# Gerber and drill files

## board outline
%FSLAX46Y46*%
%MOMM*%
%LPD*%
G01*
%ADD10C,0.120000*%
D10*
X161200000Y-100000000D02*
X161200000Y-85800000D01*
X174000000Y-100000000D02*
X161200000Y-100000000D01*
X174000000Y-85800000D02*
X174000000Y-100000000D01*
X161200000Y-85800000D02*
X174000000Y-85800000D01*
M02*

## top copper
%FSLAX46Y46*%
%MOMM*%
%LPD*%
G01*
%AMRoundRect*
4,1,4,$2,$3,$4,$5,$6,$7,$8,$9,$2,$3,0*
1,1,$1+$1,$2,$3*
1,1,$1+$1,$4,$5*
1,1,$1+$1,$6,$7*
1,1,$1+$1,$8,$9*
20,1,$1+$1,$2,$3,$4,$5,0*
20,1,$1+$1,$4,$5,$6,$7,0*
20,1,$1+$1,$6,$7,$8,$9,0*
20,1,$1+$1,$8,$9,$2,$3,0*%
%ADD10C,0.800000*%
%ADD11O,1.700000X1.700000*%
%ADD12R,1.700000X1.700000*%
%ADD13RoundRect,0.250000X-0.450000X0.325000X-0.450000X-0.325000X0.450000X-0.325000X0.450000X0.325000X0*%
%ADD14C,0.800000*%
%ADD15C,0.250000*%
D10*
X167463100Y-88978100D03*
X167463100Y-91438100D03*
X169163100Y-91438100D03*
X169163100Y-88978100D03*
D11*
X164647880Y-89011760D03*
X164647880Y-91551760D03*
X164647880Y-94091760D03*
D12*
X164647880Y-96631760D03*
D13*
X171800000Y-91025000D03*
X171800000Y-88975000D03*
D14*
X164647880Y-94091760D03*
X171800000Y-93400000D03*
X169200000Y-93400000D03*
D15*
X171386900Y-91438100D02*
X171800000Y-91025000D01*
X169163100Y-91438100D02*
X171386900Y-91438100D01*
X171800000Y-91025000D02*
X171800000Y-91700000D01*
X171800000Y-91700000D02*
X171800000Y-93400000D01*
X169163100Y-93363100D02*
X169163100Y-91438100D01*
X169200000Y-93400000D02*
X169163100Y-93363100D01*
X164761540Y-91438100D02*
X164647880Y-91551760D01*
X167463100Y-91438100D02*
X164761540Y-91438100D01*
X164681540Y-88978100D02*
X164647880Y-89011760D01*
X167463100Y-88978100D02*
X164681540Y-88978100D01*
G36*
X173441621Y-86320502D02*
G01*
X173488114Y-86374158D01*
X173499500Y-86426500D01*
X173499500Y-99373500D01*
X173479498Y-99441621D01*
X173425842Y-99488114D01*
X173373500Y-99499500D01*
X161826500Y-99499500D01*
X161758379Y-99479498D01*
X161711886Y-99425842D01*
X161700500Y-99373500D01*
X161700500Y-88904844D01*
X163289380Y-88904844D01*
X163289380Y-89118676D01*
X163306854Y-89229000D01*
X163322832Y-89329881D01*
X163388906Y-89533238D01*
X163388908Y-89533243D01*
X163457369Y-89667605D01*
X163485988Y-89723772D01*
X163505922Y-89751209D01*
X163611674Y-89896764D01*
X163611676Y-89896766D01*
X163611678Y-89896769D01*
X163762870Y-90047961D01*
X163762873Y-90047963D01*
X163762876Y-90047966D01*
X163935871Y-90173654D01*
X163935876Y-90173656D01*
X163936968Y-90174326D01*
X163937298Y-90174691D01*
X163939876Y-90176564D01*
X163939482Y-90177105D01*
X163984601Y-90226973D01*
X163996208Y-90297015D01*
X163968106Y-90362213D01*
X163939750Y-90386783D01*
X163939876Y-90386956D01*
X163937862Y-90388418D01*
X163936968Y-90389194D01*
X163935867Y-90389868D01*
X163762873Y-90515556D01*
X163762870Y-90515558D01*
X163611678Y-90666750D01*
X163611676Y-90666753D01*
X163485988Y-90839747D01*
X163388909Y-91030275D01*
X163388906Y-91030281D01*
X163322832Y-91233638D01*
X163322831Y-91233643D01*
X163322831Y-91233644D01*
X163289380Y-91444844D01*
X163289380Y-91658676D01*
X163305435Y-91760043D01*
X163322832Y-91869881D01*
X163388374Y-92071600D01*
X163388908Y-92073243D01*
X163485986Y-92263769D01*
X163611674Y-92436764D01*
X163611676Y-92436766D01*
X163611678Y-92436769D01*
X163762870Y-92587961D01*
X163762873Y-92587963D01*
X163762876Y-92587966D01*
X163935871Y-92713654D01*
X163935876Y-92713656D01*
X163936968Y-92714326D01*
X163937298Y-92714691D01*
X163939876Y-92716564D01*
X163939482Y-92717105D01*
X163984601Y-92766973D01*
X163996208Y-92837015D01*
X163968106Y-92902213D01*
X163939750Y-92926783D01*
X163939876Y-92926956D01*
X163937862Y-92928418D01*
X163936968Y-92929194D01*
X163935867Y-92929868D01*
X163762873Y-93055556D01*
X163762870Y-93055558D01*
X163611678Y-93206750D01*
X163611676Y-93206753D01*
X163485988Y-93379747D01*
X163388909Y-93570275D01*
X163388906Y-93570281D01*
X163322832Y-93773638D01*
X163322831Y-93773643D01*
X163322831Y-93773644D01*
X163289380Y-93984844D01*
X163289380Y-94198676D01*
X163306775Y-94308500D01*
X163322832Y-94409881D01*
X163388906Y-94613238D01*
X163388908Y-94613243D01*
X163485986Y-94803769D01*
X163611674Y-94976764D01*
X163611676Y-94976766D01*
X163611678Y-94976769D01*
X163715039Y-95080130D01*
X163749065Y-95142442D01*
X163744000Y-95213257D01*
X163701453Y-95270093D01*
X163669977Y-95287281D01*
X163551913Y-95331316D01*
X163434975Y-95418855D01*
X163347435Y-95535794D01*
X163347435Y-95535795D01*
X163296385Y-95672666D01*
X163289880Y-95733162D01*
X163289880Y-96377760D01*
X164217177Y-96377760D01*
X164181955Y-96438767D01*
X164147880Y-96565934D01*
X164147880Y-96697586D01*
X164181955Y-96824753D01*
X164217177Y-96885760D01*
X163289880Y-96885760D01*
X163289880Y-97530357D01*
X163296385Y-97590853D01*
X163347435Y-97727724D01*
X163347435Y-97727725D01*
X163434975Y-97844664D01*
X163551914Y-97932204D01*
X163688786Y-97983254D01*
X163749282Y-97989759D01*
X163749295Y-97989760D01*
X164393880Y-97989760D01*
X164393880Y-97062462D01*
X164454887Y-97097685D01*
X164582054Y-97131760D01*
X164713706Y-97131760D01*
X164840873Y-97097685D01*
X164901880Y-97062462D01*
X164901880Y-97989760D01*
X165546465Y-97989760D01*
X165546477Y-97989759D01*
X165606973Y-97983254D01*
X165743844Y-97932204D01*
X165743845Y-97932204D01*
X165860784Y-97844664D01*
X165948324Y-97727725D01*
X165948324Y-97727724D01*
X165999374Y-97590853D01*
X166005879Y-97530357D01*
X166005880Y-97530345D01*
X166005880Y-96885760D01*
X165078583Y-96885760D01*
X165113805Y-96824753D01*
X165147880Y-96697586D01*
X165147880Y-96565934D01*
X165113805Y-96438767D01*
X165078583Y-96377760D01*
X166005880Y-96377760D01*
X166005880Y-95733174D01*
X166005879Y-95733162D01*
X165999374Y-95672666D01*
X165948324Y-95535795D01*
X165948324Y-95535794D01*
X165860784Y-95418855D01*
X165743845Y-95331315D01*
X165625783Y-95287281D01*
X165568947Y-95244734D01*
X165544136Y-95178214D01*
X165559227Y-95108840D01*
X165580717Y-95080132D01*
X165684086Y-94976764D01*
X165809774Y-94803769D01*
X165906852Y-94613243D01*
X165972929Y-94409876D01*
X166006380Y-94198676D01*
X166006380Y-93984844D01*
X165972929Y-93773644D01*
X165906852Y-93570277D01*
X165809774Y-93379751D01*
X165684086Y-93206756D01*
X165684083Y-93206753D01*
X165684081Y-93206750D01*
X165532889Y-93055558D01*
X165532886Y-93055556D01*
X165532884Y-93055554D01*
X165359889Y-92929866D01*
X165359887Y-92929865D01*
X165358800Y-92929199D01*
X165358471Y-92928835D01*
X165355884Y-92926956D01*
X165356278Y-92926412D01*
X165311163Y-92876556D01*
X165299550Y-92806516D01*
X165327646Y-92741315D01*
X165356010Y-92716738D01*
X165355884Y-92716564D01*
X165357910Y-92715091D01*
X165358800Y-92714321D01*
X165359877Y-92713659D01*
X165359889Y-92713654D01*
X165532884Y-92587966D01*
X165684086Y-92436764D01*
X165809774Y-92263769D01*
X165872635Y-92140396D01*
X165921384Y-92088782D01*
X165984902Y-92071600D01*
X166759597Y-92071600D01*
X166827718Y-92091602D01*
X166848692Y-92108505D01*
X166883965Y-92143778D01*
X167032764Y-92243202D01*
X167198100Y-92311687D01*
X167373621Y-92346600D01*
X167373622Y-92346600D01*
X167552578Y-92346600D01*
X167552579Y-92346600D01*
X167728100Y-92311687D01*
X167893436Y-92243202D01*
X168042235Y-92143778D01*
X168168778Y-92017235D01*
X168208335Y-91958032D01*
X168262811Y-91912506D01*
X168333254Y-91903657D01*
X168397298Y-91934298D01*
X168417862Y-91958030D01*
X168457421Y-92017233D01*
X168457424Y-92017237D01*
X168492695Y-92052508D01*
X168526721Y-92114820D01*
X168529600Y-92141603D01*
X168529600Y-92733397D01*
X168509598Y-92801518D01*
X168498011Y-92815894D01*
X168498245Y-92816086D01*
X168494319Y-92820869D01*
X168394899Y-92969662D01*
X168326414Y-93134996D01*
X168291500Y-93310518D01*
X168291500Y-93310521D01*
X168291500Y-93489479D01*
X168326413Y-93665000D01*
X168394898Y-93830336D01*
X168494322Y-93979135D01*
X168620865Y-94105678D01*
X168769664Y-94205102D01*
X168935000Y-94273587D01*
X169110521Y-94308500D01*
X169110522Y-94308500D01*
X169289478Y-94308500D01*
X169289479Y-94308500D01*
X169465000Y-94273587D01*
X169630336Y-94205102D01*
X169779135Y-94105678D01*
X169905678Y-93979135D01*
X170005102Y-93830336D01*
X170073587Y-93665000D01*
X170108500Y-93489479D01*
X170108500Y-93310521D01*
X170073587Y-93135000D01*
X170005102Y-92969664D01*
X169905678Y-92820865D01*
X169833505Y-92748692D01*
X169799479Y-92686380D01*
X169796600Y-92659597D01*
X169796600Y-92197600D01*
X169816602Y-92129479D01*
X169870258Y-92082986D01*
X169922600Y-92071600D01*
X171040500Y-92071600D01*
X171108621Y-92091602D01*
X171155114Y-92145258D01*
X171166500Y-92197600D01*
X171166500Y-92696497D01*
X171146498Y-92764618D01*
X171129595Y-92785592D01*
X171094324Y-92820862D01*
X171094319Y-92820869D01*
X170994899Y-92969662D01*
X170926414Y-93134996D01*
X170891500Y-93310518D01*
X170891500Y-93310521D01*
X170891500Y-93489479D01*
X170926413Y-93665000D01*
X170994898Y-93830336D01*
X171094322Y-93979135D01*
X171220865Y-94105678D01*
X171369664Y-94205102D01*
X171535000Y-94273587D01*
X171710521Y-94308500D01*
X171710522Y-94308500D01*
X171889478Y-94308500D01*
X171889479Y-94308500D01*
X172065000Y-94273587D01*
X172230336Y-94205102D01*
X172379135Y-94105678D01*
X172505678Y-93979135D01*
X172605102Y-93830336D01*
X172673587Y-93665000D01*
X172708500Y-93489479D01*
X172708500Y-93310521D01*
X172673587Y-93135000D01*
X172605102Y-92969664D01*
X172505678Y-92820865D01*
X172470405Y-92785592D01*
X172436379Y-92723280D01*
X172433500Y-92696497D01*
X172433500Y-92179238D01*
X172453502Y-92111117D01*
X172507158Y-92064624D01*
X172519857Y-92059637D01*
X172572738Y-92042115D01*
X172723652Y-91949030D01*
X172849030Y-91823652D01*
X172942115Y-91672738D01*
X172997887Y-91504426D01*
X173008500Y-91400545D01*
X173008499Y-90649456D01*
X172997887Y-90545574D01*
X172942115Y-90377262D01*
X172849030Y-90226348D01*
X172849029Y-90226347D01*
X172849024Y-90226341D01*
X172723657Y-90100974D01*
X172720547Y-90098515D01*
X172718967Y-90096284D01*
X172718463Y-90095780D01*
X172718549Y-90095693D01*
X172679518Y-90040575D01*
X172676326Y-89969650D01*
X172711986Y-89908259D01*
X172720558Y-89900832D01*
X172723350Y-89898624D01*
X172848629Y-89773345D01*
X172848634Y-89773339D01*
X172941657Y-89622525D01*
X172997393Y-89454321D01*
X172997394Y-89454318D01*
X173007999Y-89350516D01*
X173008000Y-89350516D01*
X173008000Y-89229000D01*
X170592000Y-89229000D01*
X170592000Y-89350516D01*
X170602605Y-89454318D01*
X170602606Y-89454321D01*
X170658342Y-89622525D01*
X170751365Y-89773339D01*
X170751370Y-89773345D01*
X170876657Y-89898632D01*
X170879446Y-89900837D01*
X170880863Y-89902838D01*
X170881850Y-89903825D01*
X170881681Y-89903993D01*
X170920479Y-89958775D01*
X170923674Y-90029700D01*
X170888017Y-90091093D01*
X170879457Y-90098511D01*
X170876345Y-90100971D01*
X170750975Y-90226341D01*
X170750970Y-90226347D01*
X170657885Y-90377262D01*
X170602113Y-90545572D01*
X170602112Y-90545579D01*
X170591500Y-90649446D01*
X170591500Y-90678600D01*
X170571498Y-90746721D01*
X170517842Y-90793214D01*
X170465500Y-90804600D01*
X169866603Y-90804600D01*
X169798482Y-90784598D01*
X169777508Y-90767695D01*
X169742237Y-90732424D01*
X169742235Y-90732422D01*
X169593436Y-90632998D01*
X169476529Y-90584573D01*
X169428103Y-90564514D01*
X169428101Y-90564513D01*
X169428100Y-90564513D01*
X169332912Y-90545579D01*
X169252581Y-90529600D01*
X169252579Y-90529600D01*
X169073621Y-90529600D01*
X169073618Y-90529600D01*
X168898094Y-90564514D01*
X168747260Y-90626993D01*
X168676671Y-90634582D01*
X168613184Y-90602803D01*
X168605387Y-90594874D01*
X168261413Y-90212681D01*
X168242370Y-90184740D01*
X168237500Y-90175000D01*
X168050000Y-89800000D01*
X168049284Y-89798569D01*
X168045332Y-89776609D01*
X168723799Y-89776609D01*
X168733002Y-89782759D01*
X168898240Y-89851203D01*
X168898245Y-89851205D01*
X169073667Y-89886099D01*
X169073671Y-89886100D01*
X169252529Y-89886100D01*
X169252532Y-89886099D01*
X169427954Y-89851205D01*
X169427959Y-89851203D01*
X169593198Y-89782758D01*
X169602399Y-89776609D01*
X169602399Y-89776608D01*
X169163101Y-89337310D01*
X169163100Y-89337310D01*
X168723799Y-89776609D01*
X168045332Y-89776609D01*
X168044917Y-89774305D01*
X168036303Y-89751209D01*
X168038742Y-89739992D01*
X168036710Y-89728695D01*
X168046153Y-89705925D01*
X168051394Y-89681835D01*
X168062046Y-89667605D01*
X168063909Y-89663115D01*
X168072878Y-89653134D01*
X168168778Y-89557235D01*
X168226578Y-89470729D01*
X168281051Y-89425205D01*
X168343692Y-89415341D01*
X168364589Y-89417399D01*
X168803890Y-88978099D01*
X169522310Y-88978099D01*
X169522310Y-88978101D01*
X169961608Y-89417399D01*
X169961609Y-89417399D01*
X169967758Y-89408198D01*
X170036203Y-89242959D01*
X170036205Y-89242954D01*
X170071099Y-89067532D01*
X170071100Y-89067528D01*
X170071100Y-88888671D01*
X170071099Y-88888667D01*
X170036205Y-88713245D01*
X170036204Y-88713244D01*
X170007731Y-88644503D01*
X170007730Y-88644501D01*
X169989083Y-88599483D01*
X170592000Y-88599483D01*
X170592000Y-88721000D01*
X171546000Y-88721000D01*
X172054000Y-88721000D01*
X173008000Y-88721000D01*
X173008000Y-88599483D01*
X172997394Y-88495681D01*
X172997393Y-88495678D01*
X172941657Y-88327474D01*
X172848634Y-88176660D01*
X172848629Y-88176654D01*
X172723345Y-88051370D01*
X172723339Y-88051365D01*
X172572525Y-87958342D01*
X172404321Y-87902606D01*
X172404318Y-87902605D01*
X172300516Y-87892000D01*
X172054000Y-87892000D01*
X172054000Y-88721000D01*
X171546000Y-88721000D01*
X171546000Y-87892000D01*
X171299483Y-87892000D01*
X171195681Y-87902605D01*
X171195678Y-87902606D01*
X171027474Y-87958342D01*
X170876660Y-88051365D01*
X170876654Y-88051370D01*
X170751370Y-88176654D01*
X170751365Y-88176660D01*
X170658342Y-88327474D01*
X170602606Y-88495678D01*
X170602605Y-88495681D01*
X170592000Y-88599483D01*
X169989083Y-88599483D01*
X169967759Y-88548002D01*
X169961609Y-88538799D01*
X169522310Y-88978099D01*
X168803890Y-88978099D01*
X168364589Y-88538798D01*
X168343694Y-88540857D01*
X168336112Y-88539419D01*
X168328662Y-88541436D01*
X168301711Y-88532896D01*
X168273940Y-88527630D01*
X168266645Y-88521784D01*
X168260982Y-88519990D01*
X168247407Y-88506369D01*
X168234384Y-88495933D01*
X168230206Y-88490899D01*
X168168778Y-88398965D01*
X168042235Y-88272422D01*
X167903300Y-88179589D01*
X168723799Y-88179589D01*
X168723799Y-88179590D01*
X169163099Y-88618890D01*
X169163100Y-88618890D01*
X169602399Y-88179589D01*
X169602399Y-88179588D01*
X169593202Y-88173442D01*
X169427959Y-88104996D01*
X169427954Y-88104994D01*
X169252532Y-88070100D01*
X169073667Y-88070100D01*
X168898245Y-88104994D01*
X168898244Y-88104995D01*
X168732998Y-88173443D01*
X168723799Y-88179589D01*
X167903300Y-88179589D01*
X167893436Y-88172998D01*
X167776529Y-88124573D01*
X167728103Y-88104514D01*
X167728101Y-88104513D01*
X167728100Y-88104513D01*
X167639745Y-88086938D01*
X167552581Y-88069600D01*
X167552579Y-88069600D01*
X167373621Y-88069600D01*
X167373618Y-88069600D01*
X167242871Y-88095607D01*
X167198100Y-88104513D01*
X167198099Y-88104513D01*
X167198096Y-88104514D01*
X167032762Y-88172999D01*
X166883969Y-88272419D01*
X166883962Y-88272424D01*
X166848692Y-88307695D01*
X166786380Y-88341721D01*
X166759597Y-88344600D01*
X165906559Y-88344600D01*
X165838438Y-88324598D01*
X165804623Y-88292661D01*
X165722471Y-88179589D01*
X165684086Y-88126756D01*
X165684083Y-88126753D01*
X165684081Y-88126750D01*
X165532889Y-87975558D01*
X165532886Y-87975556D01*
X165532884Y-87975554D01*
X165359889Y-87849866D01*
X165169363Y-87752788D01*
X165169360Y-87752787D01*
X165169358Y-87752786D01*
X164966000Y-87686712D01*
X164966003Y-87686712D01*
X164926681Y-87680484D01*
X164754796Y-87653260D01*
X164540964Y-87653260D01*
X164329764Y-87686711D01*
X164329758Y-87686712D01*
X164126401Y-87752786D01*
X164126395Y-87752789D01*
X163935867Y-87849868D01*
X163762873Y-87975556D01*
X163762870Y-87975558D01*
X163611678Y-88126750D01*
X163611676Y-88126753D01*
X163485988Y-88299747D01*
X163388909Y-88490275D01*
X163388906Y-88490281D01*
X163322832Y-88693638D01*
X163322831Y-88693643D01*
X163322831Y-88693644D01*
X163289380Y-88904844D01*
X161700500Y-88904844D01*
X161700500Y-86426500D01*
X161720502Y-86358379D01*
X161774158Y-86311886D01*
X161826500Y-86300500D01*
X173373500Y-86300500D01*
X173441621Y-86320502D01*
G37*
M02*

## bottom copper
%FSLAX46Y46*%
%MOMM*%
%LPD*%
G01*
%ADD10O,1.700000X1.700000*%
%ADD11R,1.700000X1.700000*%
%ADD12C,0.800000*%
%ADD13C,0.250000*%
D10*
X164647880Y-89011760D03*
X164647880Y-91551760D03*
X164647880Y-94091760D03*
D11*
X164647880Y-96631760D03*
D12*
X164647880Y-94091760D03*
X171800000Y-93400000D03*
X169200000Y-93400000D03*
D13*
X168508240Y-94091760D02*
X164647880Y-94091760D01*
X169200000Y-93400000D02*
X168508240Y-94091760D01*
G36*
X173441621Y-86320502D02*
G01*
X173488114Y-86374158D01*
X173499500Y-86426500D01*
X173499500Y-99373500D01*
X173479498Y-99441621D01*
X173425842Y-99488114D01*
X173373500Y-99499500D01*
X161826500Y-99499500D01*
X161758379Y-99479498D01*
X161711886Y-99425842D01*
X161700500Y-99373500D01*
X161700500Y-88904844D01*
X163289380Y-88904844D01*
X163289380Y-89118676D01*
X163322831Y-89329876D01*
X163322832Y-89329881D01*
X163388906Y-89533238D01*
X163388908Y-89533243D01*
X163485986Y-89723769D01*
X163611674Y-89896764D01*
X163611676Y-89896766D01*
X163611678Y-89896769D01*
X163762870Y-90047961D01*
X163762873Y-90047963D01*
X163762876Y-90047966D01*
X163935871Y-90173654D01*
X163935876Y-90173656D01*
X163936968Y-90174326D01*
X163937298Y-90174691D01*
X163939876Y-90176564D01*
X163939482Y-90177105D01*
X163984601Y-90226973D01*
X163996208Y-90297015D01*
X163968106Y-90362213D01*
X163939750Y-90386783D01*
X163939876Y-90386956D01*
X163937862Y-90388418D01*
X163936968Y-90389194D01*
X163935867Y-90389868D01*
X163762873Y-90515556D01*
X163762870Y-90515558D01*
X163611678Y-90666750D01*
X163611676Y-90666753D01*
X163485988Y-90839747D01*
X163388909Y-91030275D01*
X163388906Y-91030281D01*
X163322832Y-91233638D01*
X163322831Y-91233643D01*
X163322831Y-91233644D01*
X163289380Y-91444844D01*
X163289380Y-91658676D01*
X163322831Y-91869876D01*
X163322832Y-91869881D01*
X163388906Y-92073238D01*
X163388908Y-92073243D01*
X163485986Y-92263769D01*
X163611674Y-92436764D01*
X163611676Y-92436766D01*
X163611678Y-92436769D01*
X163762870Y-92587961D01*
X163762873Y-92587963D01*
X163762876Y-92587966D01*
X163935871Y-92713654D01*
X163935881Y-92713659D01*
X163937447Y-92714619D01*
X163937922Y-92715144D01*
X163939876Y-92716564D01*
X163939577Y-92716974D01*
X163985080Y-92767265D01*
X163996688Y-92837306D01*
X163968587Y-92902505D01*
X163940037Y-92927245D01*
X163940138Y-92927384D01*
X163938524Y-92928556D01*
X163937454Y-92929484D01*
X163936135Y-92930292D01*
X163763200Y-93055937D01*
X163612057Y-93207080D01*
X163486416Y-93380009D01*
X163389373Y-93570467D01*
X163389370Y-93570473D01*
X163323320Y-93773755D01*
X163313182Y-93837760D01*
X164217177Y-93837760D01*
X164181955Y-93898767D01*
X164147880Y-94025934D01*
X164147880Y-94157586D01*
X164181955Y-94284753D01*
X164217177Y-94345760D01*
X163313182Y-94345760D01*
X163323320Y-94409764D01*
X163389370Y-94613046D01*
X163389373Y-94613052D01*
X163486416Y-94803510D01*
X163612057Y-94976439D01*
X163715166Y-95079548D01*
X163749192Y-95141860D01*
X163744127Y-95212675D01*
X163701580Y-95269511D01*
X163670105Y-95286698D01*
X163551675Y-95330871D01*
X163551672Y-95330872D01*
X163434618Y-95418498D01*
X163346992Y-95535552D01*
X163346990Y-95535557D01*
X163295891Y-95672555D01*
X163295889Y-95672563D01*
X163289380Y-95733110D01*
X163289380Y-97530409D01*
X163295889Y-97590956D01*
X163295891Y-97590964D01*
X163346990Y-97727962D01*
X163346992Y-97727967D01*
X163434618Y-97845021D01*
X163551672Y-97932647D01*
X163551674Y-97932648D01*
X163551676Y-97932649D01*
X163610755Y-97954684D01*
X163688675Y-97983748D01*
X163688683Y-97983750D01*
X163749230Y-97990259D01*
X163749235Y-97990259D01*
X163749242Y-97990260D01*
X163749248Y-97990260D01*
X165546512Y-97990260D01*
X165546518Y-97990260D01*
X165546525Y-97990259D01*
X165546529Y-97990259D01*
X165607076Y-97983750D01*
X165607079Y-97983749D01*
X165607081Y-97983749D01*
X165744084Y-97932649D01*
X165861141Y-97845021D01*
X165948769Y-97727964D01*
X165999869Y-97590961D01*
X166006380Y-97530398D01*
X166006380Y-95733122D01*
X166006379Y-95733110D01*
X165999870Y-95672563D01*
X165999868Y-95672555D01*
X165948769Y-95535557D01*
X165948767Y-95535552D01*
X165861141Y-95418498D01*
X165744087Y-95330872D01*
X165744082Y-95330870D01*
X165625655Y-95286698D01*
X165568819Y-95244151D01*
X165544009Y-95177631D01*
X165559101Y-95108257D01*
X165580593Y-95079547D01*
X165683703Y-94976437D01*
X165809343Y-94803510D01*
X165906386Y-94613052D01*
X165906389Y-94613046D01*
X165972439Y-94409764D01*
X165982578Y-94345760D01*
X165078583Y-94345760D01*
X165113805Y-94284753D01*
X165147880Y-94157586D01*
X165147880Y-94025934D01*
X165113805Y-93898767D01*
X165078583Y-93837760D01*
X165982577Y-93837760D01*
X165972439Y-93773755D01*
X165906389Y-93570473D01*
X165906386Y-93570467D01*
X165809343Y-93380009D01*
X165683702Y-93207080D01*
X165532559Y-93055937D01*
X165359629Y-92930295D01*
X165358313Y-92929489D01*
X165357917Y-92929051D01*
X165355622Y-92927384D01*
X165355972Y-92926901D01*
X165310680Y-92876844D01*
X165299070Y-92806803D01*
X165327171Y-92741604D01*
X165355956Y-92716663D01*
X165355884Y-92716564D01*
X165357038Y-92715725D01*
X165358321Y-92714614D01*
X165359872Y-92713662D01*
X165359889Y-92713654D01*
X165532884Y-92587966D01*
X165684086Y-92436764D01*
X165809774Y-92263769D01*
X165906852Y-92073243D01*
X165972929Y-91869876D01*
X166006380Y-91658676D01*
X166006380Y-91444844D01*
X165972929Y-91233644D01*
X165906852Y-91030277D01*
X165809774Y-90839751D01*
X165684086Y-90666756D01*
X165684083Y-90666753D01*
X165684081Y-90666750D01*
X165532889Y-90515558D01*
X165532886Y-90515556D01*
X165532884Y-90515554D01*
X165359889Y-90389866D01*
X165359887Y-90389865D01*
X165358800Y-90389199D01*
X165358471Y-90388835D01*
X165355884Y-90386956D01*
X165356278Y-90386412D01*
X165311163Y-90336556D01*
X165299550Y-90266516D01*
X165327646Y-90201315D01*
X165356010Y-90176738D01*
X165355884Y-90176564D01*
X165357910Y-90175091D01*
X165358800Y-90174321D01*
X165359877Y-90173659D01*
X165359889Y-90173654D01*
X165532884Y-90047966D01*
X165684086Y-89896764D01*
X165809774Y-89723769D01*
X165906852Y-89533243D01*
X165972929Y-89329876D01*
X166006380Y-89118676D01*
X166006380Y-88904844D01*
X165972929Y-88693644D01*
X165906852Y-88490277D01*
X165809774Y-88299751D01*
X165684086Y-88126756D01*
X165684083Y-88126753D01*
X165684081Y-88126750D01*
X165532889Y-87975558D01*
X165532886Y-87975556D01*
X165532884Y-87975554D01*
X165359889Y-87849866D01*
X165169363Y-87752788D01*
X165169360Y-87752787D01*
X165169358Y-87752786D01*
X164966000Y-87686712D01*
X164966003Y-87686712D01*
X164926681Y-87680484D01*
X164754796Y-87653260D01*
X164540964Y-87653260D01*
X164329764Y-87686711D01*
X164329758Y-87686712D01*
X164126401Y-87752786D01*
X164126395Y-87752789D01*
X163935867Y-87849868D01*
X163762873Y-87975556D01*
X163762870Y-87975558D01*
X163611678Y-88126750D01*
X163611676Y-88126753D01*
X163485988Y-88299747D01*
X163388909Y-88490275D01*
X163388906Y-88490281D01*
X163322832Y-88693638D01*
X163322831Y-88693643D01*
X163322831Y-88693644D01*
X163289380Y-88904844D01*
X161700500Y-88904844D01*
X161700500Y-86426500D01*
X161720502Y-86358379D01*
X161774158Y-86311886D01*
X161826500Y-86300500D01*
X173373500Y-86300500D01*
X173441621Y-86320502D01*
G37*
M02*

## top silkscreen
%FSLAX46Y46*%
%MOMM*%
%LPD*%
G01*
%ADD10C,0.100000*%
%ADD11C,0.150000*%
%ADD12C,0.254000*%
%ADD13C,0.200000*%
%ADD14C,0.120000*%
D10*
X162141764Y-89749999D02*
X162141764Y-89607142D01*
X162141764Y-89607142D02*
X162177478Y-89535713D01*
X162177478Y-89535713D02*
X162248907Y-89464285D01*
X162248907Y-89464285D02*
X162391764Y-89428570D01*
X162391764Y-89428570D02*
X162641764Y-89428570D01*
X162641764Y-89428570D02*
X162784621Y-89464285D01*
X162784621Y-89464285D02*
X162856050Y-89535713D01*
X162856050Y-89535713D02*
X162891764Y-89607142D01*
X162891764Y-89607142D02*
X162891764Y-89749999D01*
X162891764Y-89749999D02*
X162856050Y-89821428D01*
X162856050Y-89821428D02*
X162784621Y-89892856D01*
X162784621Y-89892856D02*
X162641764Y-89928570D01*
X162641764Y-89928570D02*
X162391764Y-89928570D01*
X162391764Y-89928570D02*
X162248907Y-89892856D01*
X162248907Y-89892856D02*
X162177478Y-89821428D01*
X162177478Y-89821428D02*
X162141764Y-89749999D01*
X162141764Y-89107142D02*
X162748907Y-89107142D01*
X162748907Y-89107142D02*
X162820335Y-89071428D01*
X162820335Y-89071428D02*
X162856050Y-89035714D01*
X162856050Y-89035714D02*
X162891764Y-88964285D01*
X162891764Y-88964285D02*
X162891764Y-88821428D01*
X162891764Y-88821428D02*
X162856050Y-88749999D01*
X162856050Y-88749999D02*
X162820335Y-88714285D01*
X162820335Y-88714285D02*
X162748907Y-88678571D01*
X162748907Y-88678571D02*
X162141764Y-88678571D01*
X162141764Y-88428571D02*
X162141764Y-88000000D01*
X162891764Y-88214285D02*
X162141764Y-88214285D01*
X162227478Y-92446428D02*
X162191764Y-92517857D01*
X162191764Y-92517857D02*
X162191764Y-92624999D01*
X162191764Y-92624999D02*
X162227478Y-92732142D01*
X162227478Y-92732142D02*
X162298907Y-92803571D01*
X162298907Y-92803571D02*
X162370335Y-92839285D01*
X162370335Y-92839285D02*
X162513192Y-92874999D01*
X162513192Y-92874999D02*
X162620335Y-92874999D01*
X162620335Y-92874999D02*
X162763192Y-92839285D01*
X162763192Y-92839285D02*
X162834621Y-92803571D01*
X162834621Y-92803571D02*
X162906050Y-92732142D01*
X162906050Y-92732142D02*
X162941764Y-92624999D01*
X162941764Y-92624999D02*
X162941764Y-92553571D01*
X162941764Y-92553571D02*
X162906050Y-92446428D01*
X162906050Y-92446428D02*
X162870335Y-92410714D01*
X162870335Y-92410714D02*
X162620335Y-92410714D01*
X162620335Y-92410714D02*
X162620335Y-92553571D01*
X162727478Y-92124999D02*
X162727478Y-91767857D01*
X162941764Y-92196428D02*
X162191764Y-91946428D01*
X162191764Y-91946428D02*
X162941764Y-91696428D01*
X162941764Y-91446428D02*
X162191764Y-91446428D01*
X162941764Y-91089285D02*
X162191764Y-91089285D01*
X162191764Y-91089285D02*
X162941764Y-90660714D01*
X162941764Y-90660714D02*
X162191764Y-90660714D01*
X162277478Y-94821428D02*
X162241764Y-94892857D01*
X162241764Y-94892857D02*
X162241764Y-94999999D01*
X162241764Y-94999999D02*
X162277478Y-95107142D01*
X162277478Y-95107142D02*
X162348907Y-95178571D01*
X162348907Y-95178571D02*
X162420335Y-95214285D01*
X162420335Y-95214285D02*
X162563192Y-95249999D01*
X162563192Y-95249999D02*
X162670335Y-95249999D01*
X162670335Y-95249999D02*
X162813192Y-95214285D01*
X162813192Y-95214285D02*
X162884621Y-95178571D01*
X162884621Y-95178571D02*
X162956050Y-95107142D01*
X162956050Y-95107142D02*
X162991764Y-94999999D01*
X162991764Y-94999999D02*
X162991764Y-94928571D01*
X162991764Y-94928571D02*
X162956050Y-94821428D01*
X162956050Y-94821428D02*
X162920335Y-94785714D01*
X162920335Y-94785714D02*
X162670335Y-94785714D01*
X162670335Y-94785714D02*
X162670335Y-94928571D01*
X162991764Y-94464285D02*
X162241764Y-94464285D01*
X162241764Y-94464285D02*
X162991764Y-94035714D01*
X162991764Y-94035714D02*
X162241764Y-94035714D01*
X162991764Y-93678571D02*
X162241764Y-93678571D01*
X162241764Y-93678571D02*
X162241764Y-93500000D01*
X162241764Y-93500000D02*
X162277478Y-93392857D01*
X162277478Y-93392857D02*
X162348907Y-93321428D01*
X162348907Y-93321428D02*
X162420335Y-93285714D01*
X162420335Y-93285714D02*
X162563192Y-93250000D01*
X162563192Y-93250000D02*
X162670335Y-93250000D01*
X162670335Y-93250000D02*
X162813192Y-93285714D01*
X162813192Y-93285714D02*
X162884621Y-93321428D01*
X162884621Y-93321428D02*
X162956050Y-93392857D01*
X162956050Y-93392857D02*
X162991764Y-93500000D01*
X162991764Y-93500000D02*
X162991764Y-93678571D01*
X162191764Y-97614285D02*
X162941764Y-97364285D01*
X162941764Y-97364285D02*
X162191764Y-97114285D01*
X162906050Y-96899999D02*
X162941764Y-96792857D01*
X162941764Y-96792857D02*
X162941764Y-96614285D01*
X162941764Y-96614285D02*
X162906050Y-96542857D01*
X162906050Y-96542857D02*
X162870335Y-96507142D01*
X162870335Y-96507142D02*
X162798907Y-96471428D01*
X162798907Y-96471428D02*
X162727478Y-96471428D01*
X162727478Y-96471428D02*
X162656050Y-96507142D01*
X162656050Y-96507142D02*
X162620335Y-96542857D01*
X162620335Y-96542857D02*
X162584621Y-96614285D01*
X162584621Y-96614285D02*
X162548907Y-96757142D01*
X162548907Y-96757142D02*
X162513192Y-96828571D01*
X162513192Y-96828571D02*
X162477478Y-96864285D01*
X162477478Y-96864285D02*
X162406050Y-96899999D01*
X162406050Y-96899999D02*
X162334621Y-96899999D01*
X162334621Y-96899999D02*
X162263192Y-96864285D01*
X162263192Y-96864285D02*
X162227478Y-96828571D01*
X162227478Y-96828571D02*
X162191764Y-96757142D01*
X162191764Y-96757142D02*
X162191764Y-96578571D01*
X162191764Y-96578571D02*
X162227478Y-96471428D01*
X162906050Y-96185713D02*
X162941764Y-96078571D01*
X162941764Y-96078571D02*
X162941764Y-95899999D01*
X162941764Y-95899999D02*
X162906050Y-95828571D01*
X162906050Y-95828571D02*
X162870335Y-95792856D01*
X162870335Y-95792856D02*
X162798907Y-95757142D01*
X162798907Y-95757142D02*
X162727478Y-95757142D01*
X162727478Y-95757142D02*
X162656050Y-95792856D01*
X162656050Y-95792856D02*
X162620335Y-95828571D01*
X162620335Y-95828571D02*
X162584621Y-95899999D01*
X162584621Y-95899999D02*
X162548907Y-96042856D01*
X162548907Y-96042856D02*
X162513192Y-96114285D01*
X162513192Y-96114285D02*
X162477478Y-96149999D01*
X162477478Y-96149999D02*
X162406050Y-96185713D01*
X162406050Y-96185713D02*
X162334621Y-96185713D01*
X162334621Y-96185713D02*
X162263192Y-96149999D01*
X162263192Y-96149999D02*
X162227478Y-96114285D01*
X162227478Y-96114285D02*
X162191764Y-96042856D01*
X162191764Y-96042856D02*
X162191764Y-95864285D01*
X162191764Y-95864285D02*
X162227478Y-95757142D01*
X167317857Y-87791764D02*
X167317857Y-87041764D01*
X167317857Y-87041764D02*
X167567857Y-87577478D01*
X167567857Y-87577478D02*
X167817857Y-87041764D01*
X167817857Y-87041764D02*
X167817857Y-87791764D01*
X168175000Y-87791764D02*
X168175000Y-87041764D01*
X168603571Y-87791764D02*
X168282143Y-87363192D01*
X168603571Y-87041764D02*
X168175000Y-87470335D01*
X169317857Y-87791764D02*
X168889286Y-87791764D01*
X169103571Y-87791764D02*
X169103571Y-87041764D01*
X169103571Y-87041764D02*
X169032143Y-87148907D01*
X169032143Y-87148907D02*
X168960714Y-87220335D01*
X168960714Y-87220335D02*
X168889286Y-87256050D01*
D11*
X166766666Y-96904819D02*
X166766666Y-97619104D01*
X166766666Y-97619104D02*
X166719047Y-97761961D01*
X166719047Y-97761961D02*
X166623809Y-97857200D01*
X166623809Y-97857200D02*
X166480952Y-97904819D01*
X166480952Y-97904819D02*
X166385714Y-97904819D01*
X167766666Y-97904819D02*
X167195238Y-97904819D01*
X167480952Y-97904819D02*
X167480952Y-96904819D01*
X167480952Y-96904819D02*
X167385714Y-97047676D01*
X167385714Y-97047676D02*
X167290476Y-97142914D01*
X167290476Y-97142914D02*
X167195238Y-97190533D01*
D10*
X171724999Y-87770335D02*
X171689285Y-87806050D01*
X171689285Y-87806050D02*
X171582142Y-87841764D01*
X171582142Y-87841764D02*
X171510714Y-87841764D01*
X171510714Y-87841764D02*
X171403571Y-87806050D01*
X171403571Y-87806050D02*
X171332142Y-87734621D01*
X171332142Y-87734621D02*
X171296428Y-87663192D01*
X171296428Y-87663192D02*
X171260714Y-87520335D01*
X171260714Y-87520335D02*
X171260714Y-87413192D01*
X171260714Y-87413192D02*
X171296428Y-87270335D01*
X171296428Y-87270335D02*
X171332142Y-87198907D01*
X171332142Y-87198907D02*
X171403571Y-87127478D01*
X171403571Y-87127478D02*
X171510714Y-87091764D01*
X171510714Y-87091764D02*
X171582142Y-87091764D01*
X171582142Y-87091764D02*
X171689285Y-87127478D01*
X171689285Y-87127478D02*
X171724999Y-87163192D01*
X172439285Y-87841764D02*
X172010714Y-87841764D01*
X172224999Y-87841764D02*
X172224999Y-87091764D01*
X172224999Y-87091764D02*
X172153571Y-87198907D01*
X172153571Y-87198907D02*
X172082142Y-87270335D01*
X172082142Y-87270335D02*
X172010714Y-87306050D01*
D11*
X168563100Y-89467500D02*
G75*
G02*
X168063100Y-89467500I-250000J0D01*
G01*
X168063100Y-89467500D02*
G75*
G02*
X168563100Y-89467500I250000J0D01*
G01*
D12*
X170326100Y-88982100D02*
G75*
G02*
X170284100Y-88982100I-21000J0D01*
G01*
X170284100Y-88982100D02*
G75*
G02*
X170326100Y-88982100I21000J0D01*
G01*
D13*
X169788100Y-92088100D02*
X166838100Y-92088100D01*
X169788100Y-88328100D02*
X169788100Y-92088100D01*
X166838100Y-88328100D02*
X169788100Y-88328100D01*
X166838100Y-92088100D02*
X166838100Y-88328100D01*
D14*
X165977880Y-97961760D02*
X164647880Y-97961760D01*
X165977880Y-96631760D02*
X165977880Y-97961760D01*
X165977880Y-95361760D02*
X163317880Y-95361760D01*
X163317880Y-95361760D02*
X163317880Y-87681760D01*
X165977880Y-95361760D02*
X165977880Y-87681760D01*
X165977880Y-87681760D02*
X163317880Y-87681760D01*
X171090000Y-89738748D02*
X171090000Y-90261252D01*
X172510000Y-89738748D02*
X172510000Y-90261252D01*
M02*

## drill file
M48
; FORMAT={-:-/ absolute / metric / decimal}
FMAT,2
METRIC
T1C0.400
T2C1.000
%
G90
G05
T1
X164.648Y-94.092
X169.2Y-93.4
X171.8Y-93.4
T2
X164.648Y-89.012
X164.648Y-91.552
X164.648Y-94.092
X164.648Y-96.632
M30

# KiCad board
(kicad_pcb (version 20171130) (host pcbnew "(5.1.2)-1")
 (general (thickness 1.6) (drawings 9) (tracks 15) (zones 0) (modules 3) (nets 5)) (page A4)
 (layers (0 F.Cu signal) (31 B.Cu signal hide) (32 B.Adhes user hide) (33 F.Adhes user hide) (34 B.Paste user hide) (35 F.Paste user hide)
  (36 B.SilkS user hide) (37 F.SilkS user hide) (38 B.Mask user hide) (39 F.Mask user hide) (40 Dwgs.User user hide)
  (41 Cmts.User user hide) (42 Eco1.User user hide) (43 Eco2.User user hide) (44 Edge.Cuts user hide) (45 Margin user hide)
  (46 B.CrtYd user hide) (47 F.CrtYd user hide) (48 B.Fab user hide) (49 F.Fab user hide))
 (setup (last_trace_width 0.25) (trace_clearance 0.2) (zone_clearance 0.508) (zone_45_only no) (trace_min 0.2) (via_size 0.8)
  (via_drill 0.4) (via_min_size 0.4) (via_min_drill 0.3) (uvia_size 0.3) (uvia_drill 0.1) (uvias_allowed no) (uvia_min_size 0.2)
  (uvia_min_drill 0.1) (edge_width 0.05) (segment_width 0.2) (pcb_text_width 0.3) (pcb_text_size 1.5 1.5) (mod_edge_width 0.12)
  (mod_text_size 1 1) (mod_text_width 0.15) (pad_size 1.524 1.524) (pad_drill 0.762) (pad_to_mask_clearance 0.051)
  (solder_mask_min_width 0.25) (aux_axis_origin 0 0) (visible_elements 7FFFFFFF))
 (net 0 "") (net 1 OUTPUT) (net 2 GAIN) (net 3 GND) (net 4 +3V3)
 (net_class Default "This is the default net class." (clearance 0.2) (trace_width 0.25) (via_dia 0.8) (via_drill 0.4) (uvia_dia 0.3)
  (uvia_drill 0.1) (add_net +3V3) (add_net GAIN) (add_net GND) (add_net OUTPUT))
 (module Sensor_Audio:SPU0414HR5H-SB (layer F.Cu) (at 168.3131 90.2081)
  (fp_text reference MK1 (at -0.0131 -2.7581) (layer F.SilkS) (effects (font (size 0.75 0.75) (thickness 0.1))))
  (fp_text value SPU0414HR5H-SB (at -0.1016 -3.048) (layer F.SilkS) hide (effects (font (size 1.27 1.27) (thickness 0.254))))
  (fp_circle (center 0 -0.7406) (end 0.25 -0.7406) (layer F.SilkS) (width 0.15))
  (fp_circle (center 1.992 -1.226) (end 1.971 -1.226) (layer F.SilkS) (width 0.254))
  (fp_line (start 1.475 1.88) (end -1.475 1.88) (layer F.SilkS) (width 0.2))
  (fp_line (start 1.475 -1.88) (end 1.475 1.88) (layer F.SilkS) (width 0.2))
  (fp_line (start -1.475 -1.88) (end 1.475 -1.88) (layer F.SilkS) (width 0.2))
  (fp_line (start -1.475 1.88) (end -1.475 -1.88) (layer F.SilkS) (width 0.2))
  (pad 4 smd circle (at -0.85 -1.23 90) (size 0.8 0.8) (layers F.Cu F.Paste F.Mask) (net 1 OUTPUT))
  (pad 3 smd circle (at -0.85 1.23 90) (size 0.8 0.8) (layers F.Cu F.Paste F.Mask) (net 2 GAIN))
  (pad 2 smd circle (at 0.85 1.23 90) (size 0.8 0.8) (layers F.Cu F.Paste F.Mask) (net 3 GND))
  (pad 1 smd circle (at 0.85 -1.23 90) (size 0.8 0.8) (layers F.Cu F.Paste F.Mask) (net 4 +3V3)))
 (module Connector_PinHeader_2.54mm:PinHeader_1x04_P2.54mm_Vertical (layer F.Cu) (at 164.64788 96.63176 180)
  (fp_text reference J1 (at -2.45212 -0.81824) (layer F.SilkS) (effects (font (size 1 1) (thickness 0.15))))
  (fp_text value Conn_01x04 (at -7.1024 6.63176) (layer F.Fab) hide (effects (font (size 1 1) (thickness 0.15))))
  (fp_line (start -1.33 -1.33) (end 0 -1.33) (layer F.SilkS) (width 0.12))
  (fp_line (start -1.33 0) (end -1.33 -1.33) (layer F.SilkS) (width 0.12))
  (fp_line (start -1.33 1.27) (end 1.33 1.27) (layer F.SilkS) (width 0.12))
  (fp_line (start 1.33 1.27) (end 1.33 8.95) (layer F.SilkS) (width 0.12))
  (fp_line (start -1.33 1.27) (end -1.33 8.95) (layer F.SilkS) (width 0.12))
  (fp_line (start -1.33 8.95) (end 1.33 8.95) (layer F.SilkS) (width 0.12))
  (pad 4 thru_hole oval (at 0 7.62 180) (size 1.7 1.7) (drill 1) (layers *.Cu *.Mask) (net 1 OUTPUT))
  (pad 3 thru_hole oval (at 0 5.08 180) (size 1.7 1.7) (drill 1) (layers *.Cu *.Mask) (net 2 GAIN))
  (pad 2 thru_hole oval (at 0 2.54 180) (size 1.7 1.7) (drill 1) (layers *.Cu *.Mask) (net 3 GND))
  (pad 1 thru_hole rect (at 0 0 180) (size 1.7 1.7) (drill 1) (layers *.Cu *.Mask) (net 4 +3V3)))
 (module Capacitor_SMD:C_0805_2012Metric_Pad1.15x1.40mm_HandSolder (layer F.Cu) (at 171.8 90 270)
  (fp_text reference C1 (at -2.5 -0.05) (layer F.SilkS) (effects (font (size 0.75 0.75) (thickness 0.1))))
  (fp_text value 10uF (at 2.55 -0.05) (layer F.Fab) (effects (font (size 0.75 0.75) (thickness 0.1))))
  (fp_line (start -0.261252 0.71) (end 0.261252 0.71) (layer F.SilkS) (width 0.12))
  (fp_line (start -0.261252 -0.71) (end 0.261252 -0.71) (layer F.SilkS) (width 0.12))
  (pad 2 smd roundrect (at 1.025 0 270) (size 1.15 1.4) (layers F.Cu F.Paste F.Mask) (roundrect_rratio 0.217391) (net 3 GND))
  (pad 1 smd roundrect (at -1.025 0 270) (size 1.15 1.4) (layers F.Cu F.Paste F.Mask) (roundrect_rratio 0.217391) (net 4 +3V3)))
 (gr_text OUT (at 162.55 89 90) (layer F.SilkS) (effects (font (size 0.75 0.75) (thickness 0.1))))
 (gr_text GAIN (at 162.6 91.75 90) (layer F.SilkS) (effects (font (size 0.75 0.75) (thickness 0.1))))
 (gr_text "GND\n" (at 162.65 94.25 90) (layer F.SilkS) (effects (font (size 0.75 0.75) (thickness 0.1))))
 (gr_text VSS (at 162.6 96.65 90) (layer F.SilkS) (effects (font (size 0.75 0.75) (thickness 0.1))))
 (gr_line (start 161.2 100) (end 161.2 85.8) (layer Edge.Cuts) (width 0.12))
 (gr_line (start 174 100) (end 161.2 100) (layer Edge.Cuts) (width 0.12))
 (gr_line (start 174 85.8) (end 174 100) (layer Edge.Cuts) (width 0.12))
 (gr_line (start 161.2 85.8) (end 174 85.8) (layer Edge.Cuts) (width 0.12))
 (via (at 164.64788 94.09176) (size 0.8) (drill 0.4) (layers F.Cu B.Cu) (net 3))
 (segment (start 171.3869 91.4381) (end 171.8 91.025) (width 0.25) (layer F.Cu) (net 3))
 (segment (start 169.1631 91.4381) (end 171.3869 91.4381) (width 0.25) (layer F.Cu) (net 3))
 (segment (start 171.8 91.025) (end 171.8 91.7) (width 0.25) (layer F.Cu) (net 3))
 (via (at 171.8 93.4) (size 0.8) (drill 0.4) (layers F.Cu B.Cu) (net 3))
 (segment (start 171.8 91.7) (end 171.8 93.4) (width 0.25) (layer F.Cu) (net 3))
 (via (at 169.2 93.4) (size 0.8) (drill 0.4) (layers F.Cu B.Cu) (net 3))
 (segment (start 168.50824 94.09176) (end 164.64788 94.09176) (width 0.25) (layer B.Cu) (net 3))
 (segment (start 169.2 93.4) (end 168.50824 94.09176) (width 0.25) (layer B.Cu) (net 3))
 (segment (start 169.1631 93.3631) (end 169.1631 91.4381) (width 0.25) (layer F.Cu) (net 3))
 (segment (start 169.2 93.4) (end 169.1631 93.3631) (width 0.25) (layer F.Cu) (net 3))
 (segment (start 164.76154 91.4381) (end 164.64788 91.55176) (width 0.25) (layer F.Cu) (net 2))
 (segment (start 167.4631 91.4381) (end 164.76154 91.4381) (width 0.25) (layer F.Cu) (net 2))
 (segment (start 164.68154 88.9781) (end 164.64788 89.01176) (width 0.25) (layer F.Cu) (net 1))
 (segment (start 167.4631 88.9781) (end 164.68154 88.9781) (width 0.25) (layer F.Cu) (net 1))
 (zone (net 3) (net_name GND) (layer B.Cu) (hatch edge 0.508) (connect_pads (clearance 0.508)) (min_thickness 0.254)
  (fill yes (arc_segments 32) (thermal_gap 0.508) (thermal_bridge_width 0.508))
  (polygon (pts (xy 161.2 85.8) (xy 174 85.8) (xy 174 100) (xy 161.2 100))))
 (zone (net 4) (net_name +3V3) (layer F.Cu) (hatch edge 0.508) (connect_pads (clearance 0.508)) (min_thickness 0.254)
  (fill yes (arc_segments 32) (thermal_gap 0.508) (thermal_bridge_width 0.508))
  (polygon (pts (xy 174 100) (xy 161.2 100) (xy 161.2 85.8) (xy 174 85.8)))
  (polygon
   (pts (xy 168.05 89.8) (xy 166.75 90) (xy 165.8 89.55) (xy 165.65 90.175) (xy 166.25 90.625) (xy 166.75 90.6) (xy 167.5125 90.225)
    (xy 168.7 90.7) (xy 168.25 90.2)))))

